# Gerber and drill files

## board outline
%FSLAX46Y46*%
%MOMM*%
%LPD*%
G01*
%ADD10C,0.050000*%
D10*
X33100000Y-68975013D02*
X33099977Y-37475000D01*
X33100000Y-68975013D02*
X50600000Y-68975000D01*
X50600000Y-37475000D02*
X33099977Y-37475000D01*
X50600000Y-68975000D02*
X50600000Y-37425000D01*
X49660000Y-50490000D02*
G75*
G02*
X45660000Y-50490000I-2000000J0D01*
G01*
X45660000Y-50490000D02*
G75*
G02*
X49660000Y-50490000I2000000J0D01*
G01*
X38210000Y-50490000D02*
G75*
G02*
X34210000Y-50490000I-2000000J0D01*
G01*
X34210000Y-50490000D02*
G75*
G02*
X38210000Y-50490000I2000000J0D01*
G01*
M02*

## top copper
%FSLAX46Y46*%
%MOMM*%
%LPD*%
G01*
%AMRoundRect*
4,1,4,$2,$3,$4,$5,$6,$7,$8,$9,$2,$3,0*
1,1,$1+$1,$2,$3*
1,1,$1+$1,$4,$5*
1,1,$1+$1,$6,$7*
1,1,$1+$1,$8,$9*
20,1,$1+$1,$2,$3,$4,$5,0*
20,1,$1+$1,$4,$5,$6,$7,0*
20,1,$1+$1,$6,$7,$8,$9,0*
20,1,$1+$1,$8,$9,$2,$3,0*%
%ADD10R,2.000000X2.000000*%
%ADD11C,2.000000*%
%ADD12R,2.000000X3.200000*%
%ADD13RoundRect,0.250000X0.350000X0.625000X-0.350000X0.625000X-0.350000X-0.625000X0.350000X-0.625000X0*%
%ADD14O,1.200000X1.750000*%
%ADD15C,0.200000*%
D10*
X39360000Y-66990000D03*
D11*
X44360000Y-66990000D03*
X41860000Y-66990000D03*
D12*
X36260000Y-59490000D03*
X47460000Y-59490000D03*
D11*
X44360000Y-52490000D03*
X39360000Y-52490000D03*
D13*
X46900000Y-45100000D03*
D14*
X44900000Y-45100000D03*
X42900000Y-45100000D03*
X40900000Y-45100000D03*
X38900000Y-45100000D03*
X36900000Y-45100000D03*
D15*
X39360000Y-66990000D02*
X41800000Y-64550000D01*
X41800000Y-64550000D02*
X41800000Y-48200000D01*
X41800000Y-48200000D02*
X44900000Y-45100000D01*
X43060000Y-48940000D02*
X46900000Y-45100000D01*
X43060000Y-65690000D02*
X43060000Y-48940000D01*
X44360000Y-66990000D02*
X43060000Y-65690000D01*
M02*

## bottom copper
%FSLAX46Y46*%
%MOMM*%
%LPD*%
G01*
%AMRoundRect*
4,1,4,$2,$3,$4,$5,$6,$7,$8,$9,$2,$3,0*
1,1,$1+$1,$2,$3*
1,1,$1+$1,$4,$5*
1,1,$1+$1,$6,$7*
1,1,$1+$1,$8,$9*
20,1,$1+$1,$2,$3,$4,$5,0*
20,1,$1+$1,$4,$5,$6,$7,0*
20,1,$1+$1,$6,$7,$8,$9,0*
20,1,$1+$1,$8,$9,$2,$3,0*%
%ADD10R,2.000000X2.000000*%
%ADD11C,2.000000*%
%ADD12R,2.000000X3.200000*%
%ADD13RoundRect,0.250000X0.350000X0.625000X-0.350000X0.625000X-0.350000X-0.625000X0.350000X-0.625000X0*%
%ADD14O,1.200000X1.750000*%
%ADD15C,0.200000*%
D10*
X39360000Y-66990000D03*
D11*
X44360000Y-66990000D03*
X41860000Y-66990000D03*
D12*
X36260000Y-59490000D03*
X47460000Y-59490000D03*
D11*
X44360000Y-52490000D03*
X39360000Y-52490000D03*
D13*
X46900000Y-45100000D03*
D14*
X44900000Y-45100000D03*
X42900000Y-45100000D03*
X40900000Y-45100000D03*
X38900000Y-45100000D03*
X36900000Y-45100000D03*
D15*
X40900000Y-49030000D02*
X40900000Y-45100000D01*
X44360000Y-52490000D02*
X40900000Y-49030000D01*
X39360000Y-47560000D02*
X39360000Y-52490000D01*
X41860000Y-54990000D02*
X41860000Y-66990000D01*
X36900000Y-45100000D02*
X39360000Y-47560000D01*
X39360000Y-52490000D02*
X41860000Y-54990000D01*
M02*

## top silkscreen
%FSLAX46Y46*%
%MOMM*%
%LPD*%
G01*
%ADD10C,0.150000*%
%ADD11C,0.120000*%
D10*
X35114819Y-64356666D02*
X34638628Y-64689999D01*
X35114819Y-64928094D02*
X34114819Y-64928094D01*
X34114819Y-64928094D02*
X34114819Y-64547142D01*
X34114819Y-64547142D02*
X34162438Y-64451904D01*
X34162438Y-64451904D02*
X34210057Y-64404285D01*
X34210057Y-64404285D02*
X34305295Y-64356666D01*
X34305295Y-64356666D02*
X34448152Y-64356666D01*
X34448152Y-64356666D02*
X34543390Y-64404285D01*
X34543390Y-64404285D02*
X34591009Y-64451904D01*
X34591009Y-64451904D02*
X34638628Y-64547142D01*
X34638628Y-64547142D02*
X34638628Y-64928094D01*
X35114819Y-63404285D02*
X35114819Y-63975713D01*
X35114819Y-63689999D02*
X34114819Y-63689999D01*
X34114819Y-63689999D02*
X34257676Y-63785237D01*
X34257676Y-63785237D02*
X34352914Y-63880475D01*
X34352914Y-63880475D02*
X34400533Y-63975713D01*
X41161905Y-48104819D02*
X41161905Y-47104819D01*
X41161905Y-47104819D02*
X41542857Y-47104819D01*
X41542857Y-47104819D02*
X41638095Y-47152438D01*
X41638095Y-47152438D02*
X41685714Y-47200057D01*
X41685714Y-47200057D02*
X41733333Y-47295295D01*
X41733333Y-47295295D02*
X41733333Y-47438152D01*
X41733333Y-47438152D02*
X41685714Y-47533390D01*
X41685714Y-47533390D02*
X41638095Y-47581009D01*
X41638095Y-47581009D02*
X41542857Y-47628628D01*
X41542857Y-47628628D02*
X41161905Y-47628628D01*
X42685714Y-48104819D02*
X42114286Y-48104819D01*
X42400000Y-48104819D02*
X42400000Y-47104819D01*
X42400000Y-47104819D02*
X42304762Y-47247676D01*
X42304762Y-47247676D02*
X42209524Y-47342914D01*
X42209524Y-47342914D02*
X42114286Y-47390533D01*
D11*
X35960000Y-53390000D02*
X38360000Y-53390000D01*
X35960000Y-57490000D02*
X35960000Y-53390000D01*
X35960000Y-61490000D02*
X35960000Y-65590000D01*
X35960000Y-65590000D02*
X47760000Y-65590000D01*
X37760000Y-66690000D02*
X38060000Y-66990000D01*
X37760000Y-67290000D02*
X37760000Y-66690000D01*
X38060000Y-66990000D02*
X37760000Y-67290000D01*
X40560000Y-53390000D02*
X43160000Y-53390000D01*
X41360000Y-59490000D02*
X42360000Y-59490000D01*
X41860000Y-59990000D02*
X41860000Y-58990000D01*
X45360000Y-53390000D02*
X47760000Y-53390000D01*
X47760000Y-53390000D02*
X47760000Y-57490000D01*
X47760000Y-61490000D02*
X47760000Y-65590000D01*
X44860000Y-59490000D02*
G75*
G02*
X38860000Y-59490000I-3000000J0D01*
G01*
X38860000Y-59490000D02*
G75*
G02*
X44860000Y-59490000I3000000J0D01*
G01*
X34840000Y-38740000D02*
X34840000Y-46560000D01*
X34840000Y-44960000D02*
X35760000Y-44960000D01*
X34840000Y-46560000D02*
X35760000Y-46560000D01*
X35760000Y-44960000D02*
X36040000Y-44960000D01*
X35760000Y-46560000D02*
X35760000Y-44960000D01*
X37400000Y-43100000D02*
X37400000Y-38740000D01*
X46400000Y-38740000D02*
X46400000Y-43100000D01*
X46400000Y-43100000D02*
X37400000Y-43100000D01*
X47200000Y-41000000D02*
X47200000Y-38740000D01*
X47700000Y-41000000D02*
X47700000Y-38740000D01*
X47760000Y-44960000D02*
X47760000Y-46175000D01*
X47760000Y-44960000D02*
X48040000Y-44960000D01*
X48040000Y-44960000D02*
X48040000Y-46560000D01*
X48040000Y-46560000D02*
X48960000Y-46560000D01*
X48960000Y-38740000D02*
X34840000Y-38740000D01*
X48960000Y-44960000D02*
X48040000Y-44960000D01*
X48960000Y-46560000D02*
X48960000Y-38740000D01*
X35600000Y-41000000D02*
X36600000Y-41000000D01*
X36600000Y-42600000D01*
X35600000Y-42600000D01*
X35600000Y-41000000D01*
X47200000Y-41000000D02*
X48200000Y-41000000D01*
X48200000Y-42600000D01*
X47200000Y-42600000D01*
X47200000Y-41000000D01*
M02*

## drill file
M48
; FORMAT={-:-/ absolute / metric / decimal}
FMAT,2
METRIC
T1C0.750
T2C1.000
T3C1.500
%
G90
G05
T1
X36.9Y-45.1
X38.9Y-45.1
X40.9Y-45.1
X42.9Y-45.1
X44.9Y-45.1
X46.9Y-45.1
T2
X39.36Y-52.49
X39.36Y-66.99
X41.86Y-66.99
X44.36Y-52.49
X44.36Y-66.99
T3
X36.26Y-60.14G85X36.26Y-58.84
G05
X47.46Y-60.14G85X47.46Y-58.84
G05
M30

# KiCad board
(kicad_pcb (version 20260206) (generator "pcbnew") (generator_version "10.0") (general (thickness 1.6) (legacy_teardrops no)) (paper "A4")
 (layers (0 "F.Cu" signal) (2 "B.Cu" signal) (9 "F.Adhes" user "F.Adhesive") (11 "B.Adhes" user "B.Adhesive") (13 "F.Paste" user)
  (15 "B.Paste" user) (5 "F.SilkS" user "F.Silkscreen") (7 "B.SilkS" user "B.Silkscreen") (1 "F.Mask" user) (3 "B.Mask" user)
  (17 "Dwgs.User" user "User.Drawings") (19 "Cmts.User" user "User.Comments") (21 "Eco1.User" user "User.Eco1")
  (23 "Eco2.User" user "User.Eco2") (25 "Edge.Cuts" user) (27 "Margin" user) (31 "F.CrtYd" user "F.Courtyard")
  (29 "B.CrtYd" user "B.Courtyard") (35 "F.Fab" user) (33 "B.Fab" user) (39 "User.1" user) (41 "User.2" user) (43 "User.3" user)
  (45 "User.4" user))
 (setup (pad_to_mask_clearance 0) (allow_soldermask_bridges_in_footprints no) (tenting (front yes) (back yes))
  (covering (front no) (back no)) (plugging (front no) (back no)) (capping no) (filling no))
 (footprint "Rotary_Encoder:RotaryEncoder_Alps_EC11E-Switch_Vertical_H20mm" (layer "F.Cu") (at 39.36 66.99 90)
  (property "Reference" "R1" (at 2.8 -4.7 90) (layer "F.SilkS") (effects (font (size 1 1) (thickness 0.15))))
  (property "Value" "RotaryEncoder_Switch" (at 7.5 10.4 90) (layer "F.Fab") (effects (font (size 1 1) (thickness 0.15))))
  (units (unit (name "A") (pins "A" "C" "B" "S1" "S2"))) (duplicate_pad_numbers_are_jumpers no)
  (fp_line (start 13.6 -3.4) (end 13.6 -1) (stroke (width 0.12) (type solid)) (layer "F.SilkS"))
  (fp_line (start 9.5 -3.4) (end 13.6 -3.4) (stroke (width 0.12) (type solid)) (layer "F.SilkS"))
  (fp_line (start 5.5 -3.4) (end 1.4 -3.4) (stroke (width 0.12) (type solid)) (layer "F.SilkS"))
  (fp_line (start 1.4 -3.4) (end 1.4 8.4) (stroke (width 0.12) (type solid)) (layer "F.SilkS"))
  (fp_line (start 0.3 -1.6) (end 0 -1.3) (stroke (width 0.12) (type solid)) (layer "F.SilkS"))
  (fp_line (start -0.3 -1.6) (end 0.3 -1.6) (stroke (width 0.12) (type solid)) (layer "F.SilkS"))
  (fp_line (start 0 -1.3) (end -0.3 -1.6) (stroke (width 0.12) (type solid)) (layer "F.SilkS"))
  (fp_line (start 13.6 1.2) (end 13.6 3.8) (stroke (width 0.12) (type solid)) (layer "F.SilkS"))
  (fp_line (start 7.5 2) (end 7.5 3) (stroke (width 0.12) (type solid)) (layer "F.SilkS"))
  (fp_line (start 7 2.5) (end 8 2.5) (stroke (width 0.12) (type solid)) (layer "F.SilkS"))
  (fp_line (start 13.6 6) (end 13.6 8.4) (stroke (width 0.12) (type solid)) (layer "F.SilkS"))
  (fp_line (start 13.6 8.4) (end 9.5 8.4) (stroke (width 0.12) (type solid)) (layer "F.SilkS"))
  (fp_line (start 5.5 8.4) (end 1.4 8.4) (stroke (width 0.12) (type solid)) (layer "F.SilkS"))
  (fp_circle (center 7.5 2.5) (end 10.5 2.5) (stroke (width 0.12) (type solid)) (fill no) (layer "F.SilkS"))
  (pad "A" thru_hole rect (at 0 0 90) (size 2 2) (drill 1) (layers "*.Cu" "*.Mask") (remove_unused_layers no) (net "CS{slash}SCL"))
  (pad "B" thru_hole circle (at 0 5 90) (size 2 2) (drill 1) (layers "*.Cu" "*.Mask") (remove_unused_layers no) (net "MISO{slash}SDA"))
  (pad "C" thru_hole circle (at 0 2.5 90) (size 2 2) (drill 1) (layers "*.Cu" "*.Mask") (remove_unused_layers no) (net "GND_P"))
  (pad "MP" thru_hole rect (at 7.5 -3.1 90) (size 3.2 2) (drill oval 2.8 1.5) (layers "*.Cu" "*.Mask") (remove_unused_layers no))
  (pad "MP" thru_hole rect (at 7.5 8.1 90) (size 3.2 2) (drill oval 2.8 1.5) (layers "*.Cu" "*.Mask") (remove_unused_layers no))
  (pad "S1" thru_hole circle (at 14.5 5 90) (size 2 2) (drill 1) (layers "*.Cu" "*.Mask") (remove_unused_layers no) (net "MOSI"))
  (pad "S2" thru_hole circle (at 14.5 0 90) (size 2 2) (drill 1) (layers "*.Cu" "*.Mask") (remove_unused_layers no) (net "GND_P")))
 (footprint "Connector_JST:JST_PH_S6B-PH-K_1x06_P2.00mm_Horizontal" (layer "F.Cu") (at 46.9 45.1 180)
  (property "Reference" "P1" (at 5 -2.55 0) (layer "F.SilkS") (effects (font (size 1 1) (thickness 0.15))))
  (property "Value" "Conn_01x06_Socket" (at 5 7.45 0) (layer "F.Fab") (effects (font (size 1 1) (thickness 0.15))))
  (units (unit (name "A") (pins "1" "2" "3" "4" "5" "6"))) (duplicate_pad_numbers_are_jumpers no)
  (fp_line (start 12.06 6.36) (end 12.06 -1.46) (stroke (width 0.12) (type solid)) (layer "F.SilkS"))
  (fp_line (start 12.06 0.14) (end 11.14 0.14) (stroke (width 0.12) (type solid)) (layer "F.SilkS"))
  (fp_line (start 12.06 -1.46) (end 11.14 -1.46) (stroke (width 0.12) (type solid)) (layer "F.SilkS"))
  (fp_line (start 11.14 0.14) (end 10.86 0.14) (stroke (width 0.12) (type solid)) (layer "F.SilkS"))
  (fp_line (start 11.14 -1.46) (end 11.14 0.14) (stroke (width 0.12) (type solid)) (layer "F.SilkS"))
  (fp_line (start 9.5 2) (end 9.5 6.36) (stroke (width 0.12) (type solid)) (layer "F.SilkS"))
  (fp_line (start 0.5 6.36) (end 0.5 2) (stroke (width 0.12) (type solid)) (layer "F.SilkS"))
  (fp_line (start 0.5 2) (end 9.5 2) (stroke (width 0.12) (type solid)) (layer "F.SilkS"))
  (fp_line (start -0.3 4.1) (end -0.3 6.36) (stroke (width 0.12) (type solid)) (layer "F.SilkS"))
  (fp_line (start -0.8 4.1) (end -0.8 6.36) (stroke (width 0.12) (type solid)) (layer "F.SilkS"))
  (fp_line (start -0.86 0.14) (end -0.86 -1.075) (stroke (width 0.12) (type solid)) (layer "F.SilkS"))
  (fp_line (start -0.86 0.14) (end -1.14 0.14) (stroke (width 0.12) (type solid)) (layer "F.SilkS"))
  (fp_line (start -1.14 0.14) (end -1.14 -1.46) (stroke (width 0.12) (type solid)) (layer "F.SilkS"))
  (fp_line (start -1.14 -1.46) (end -2.06 -1.46) (stroke (width 0.12) (type solid)) (layer "F.SilkS"))
  (fp_line (start -2.06 6.36) (end 12.06 6.36) (stroke (width 0.12) (type solid)) (layer "F.SilkS"))
  (fp_line (start -2.06 0.14) (end -1.14 0.14) (stroke (width 0.12) (type solid)) (layer "F.SilkS"))
  (fp_line (start -2.06 -1.46) (end -2.06 6.36) (stroke (width 0.12) (type solid)) (layer "F.SilkS"))
  (fp_rect (start 10.3 2.5) (end 11.3 4.1) (stroke (width 0.12) (type solid)) (fill no) (layer "F.SilkS"))
  (fp_rect (start -1.3 2.5) (end -0.3 4.1) (stroke (width 0.12) (type solid)) (fill no) (layer "F.SilkS"))
  (pad "1" thru_hole roundrect (at 0 0 180) (size 1.2 1.75) (drill 0.75) (layers "*.Cu" "*.Mask") (remove_unused_layers no)
   (roundrect_rratio 0.208333) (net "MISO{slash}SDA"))
  (pad "2" thru_hole oval (at 2 0 180) (size 1.2 1.75) (drill 0.75) (layers "*.Cu" "*.Mask") (remove_unused_layers no) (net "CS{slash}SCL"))
  (pad "3" thru_hole oval (at 4 0 180) (size 1.2 1.75) (drill 0.75) (layers "*.Cu" "*.Mask") (remove_unused_layers no)
   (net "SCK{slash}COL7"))
  (pad "4" thru_hole oval (at 6 0 180) (size 1.2 1.75) (drill 0.75) (layers "*.Cu" "*.Mask") (remove_unused_layers no) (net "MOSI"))
  (pad "5" thru_hole oval (at 8 0 180) (size 1.2 1.75) (drill 0.75) (layers "*.Cu" "*.Mask") (remove_unused_layers no) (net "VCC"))
  (pad "6" thru_hole oval (at 10 0 180) (size 1.2 1.75) (drill 0.75) (layers "*.Cu" "*.Mask") (remove_unused_layers no) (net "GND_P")))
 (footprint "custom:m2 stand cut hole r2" (layer "F.Cu") (at 47.66 50.49 90)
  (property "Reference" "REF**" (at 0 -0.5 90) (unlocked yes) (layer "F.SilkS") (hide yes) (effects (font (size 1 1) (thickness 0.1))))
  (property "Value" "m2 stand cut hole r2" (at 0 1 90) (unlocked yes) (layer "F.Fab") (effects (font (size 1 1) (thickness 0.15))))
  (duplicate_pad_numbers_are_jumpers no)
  (fp_circle (center 0 0) (end 2 0) (stroke (width 0.05) (type default)) (fill no) (layer "Edge.Cuts")))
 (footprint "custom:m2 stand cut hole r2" (layer "F.Cu") (at 36.21 50.49 90)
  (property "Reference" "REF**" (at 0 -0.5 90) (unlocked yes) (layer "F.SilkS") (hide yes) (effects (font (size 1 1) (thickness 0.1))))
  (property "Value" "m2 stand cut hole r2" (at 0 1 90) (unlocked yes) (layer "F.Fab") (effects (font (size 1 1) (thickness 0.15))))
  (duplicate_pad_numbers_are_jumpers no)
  (fp_circle (center 0 0) (end 2 0) (stroke (width 0.05) (type default)) (fill no) (layer "Edge.Cuts")))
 (gr_line (start 33.1 68.975013) (end 33.099977 37.475) (stroke (width 0.05) (type default)) (layer "Edge.Cuts"))
 (gr_line (start 33.1 68.975013) (end 50.6 68.975) (stroke (width 0.05) (type default)) (layer "Edge.Cuts"))
 (gr_line (start 50.6 37.475) (end 33.099977 37.475) (stroke (width 0.05) (type default)) (layer "Edge.Cuts"))
 (gr_line (start 50.6 68.975) (end 50.6 37.425) (stroke (width 0.05) (type default)) (layer "Edge.Cuts"))
 (segment (start 39.36 66.99) (end 41.8 64.55) (width 0.2) (layer "F.Cu") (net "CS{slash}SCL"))
 (segment (start 41.8 64.55) (end 41.8 48.2) (width 0.2) (layer "F.Cu") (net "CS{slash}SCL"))
 (segment (start 41.8 48.2) (end 44.9 45.1) (width 0.2) (layer "F.Cu") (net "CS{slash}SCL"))
 (segment (start 43.06 48.94) (end 46.9 45.1) (width 0.2) (layer "F.Cu") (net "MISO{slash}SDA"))
 (segment (start 43.06 65.69) (end 43.06 48.94) (width 0.2) (layer "F.Cu") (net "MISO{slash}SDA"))
 (segment (start 44.36 66.99) (end 43.06 65.69) (width 0.2) (layer "F.Cu") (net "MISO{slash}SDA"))
 (segment (start 40.9 49.03) (end 40.9 45.1) (width 0.2) (layer "B.Cu") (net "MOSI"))
 (segment (start 44.36 52.49) (end 40.9 49.03) (width 0.2) (layer "B.Cu") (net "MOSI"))
 (segment (start 39.36 47.56) (end 39.36 52.49) (width 0.2) (layer "B.Cu") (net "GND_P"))
 (segment (start 41.86 54.99) (end 41.86 66.99) (width 0.2) (layer "B.Cu") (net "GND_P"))
 (segment (start 36.9 45.1) (end 39.36 47.56) (width 0.2) (layer "B.Cu") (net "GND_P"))
 (segment (start 39.36 52.49) (end 41.86 54.99) (width 0.2) (layer "B.Cu") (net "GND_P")))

